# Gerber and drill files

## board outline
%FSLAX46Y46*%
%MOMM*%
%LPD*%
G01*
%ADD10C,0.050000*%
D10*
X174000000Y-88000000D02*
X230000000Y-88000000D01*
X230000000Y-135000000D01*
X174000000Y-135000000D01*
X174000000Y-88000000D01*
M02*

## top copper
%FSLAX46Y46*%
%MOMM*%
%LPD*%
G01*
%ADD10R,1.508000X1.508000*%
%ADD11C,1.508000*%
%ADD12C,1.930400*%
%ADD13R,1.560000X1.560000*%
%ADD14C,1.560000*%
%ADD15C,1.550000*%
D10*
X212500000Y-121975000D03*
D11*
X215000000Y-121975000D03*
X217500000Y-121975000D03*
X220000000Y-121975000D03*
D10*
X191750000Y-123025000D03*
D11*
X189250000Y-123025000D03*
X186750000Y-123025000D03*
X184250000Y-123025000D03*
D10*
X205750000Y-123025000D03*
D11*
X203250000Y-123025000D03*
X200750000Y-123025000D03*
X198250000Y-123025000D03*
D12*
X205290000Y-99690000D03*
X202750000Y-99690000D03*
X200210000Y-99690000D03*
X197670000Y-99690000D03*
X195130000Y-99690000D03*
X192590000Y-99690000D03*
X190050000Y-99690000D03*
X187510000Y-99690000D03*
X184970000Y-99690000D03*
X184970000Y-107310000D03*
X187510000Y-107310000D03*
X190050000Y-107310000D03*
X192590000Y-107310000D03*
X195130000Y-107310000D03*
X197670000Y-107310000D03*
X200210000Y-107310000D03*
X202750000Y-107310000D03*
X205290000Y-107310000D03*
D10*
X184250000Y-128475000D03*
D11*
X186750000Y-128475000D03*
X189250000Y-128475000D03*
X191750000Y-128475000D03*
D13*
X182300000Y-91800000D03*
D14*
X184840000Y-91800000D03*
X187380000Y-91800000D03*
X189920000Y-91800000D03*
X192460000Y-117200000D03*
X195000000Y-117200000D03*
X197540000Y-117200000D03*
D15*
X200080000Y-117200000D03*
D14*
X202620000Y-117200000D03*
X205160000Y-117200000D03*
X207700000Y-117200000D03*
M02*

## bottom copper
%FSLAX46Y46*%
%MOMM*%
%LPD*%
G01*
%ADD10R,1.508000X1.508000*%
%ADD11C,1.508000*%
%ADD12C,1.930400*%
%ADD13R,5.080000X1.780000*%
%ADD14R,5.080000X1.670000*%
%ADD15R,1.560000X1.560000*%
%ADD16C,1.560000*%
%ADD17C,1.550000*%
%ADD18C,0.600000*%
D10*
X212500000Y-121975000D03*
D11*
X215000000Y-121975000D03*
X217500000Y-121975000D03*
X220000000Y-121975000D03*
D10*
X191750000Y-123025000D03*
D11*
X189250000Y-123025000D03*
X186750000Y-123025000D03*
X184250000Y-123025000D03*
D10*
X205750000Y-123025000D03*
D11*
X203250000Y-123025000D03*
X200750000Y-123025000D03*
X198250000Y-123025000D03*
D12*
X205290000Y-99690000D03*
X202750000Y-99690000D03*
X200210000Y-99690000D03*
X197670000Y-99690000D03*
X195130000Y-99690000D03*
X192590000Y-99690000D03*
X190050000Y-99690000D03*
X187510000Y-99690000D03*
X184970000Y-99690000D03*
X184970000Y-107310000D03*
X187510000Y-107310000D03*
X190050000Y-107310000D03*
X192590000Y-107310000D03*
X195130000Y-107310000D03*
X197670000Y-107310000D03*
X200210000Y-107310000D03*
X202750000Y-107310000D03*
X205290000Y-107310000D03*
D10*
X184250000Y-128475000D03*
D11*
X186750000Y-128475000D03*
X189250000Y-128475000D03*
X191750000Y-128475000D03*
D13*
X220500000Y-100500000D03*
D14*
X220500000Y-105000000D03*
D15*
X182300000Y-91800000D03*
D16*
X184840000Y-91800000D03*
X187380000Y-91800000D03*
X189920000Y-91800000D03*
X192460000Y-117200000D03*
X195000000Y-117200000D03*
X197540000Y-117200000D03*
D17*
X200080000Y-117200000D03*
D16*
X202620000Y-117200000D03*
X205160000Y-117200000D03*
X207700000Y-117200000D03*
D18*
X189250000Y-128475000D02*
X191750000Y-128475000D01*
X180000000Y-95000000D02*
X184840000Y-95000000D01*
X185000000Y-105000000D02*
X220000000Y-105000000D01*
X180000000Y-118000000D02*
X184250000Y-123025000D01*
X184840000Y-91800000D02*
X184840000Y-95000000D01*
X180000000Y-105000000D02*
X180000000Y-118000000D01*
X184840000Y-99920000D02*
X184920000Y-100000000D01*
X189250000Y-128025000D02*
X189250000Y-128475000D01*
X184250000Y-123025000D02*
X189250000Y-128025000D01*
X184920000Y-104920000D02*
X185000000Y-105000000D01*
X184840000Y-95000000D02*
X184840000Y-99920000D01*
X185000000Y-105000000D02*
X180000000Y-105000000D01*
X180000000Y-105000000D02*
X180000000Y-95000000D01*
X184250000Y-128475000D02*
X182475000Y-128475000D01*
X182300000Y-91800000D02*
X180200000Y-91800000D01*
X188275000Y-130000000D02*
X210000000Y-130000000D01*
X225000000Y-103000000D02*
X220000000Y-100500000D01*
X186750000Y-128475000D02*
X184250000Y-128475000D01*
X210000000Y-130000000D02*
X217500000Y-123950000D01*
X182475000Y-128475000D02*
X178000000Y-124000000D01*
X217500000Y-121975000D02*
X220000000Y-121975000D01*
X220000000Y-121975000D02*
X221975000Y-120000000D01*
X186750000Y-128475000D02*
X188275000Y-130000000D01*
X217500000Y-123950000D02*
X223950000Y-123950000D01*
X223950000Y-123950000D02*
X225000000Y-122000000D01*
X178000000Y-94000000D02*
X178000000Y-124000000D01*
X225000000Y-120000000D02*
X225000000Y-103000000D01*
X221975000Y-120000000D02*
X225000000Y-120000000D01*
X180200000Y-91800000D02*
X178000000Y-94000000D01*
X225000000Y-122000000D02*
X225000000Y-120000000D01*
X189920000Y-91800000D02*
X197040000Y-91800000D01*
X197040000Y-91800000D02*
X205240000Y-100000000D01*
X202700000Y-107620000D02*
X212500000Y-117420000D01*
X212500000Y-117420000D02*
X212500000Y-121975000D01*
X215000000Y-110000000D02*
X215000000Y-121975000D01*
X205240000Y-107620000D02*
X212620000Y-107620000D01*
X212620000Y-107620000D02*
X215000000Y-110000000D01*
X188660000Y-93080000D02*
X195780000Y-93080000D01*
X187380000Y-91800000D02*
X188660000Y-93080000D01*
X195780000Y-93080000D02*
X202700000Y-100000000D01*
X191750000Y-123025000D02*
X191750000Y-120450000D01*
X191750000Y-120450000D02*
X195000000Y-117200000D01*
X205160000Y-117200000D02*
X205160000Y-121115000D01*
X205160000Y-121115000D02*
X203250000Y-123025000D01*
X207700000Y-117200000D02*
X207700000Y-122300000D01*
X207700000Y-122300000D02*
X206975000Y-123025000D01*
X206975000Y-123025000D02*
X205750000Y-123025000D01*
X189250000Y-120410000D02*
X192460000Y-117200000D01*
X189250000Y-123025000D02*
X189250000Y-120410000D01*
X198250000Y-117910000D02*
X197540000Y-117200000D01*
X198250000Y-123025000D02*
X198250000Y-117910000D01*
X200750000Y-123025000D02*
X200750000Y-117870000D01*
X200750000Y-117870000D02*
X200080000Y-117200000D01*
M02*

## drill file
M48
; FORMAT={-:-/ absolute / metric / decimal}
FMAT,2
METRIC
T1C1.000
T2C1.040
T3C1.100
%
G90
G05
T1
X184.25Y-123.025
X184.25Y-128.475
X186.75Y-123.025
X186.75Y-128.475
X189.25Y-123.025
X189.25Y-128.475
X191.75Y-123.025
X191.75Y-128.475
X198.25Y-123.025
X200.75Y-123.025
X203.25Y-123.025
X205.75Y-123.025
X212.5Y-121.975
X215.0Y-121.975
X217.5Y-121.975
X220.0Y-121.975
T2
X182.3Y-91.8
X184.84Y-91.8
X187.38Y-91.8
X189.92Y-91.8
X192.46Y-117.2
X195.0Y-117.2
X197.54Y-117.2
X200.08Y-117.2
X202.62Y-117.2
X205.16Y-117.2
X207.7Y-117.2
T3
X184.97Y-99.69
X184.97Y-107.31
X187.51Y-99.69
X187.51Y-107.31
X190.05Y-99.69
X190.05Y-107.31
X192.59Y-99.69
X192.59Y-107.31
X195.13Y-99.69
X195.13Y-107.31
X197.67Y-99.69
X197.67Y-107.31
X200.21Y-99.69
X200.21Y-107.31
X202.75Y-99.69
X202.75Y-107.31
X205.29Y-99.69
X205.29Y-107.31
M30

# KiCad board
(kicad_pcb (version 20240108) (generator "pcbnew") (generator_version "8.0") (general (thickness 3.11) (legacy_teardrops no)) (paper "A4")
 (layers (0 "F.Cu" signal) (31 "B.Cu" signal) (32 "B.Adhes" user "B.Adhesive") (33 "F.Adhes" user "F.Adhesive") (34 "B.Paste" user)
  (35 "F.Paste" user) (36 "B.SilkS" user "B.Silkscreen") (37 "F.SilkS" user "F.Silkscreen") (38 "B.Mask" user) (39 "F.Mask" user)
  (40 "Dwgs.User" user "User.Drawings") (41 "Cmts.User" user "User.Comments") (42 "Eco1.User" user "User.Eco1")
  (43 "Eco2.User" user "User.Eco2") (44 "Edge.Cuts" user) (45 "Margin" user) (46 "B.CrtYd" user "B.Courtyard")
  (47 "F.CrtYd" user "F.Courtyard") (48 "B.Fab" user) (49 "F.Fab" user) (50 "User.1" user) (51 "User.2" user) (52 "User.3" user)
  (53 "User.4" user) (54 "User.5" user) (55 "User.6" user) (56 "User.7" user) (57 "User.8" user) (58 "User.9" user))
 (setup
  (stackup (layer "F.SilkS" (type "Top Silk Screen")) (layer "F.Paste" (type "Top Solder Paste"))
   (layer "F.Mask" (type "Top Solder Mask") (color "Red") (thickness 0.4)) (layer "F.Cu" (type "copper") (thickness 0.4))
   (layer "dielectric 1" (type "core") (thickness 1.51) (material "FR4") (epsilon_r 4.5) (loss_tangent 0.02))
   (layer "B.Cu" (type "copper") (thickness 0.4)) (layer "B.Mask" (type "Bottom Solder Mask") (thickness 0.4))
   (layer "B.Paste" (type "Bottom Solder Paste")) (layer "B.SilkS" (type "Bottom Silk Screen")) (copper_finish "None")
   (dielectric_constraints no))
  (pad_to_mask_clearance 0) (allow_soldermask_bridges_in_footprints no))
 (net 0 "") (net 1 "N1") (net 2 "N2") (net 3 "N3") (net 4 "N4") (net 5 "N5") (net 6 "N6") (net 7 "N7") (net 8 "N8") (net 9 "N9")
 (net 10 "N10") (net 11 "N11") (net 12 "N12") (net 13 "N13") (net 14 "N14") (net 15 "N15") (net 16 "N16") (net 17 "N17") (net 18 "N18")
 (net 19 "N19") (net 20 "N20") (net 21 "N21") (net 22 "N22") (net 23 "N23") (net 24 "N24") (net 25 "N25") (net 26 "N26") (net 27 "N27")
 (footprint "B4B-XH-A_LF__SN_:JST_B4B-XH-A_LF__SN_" (layer "F.Cu") (at 216.25 122.5 180)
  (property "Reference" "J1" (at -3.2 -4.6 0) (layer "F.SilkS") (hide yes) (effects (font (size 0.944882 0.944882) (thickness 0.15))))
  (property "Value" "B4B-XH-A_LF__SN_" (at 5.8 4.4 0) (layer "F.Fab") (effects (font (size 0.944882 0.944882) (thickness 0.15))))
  (pad "1" thru_hole rect (at 3.75 0.525 180) (size 1.508 1.508) (drill 1) (layers "*.Cu" "*.Mask") (remove_unused_layers no) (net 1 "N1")
   (solder_mask_margin 0.102))
  (pad "2" thru_hole circle (at 1.25 0.525 180) (size 1.508 1.508) (drill 1) (layers "*.Cu" "*.Mask") (remove_unused_layers no) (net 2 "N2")
   (solder_mask_margin 0.102))
  (pad "3" thru_hole circle (at -1.25 0.525 180) (size 1.508 1.508) (drill 1) (layers "*.Cu" "*.Mask") (remove_unused_layers no)
   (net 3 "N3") (solder_mask_margin 0.102))
  (pad "4" thru_hole circle (at -3.75 0.525 180) (size 1.508 1.508) (drill 1) (layers "*.Cu" "*.Mask") (remove_unused_layers no)
   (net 3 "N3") (solder_mask_margin 0.102)))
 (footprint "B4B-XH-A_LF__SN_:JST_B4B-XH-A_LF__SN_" (layer "F.Cu") (at 188 122.5)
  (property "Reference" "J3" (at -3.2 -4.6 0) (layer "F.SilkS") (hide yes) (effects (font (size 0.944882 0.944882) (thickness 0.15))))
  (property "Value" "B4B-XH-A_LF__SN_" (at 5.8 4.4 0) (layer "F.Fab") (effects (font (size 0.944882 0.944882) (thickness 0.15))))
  (pad "1" thru_hole rect (at 3.75 0.525) (size 1.508 1.508) (drill 1) (layers "*.Cu" "*.Mask") (remove_unused_layers no) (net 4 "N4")
   (solder_mask_margin 0.102))
  (pad "2" thru_hole circle (at 1.25 0.525) (size 1.508 1.508) (drill 1) (layers "*.Cu" "*.Mask") (remove_unused_layers no) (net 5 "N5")
   (solder_mask_margin 0.102))
  (pad "3" thru_hole circle (at -1.25 0.525) (size 1.508 1.508) (drill 1) (layers "*.Cu" "*.Mask") (remove_unused_layers no) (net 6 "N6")
   (solder_mask_margin 0.102))
  (pad "4" thru_hole circle (at -3.75 0.525) (size 1.508 1.508) (drill 1) (layers "*.Cu" "*.Mask") (remove_unused_layers no) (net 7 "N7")
   (solder_mask_margin 0.102)))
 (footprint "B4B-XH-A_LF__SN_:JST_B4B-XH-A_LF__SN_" (layer "F.Cu") (at 202 122.5)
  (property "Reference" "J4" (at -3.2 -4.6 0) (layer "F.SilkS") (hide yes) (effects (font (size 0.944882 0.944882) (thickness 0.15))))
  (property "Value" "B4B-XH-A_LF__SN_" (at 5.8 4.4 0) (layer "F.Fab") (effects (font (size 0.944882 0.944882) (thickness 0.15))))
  (pad "1" thru_hole rect (at 3.75 0.525) (size 1.508 1.508) (drill 1) (layers "*.Cu" "*.Mask") (remove_unused_layers no) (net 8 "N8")
   (solder_mask_margin 0.102))
  (pad "2" thru_hole circle (at 1.25 0.525) (size 1.508 1.508) (drill 1) (layers "*.Cu" "*.Mask") (remove_unused_layers no) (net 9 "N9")
   (solder_mask_margin 0.102))
  (pad "3" thru_hole circle (at -1.25 0.525) (size 1.508 1.508) (drill 1) (layers "*.Cu" "*.Mask") (remove_unused_layers no) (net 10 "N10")
   (solder_mask_margin 0.102))
  (pad "4" thru_hole circle (at -3.75 0.525) (size 1.508 1.508) (drill 1) (layers "*.Cu" "*.Mask") (remove_unused_layers no) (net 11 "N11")
   (solder_mask_margin 0.102)))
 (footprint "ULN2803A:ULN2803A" (layer "F.Cu") (at 196.4 103.5 -90)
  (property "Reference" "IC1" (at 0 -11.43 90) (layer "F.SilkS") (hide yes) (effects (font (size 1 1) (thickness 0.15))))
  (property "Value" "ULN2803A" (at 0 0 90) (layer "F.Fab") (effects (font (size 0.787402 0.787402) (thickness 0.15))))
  (pad "1" thru_hole circle (at -3.81 -8.89 270) (size 1.9304 1.9304) (drill 1.1) (layers "*.Cu" "*.Mask") (remove_unused_layers no)
   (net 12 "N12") (solder_mask_margin 0.102))
  (pad "2" thru_hole circle (at -3.81 -6.35 270) (size 1.9304 1.9304) (drill 1.1) (layers "*.Cu" "*.Mask") (remove_unused_layers no)
   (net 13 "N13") (solder_mask_margin 0.102))
  (pad "3" thru_hole circle (at -3.81 -3.81 270) (size 1.9304 1.9304) (drill 1.1) (layers "*.Cu" "*.Mask") (remove_unused_layers no)
   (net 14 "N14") (solder_mask_margin 0.102))
  (pad "4" thru_hole circle (at -3.81 -1.27 270) (size 1.9304 1.9304) (drill 1.1) (layers "*.Cu" "*.Mask") (remove_unused_layers no)
   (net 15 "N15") (solder_mask_margin 0.102))
  (pad "5" thru_hole circle (at -3.81 1.27 270) (size 1.9304 1.9304) (drill 1.1) (layers "*.Cu" "*.Mask") (remove_unused_layers no)
   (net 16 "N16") (solder_mask_margin 0.102))
  (pad "6" thru_hole circle (at -3.81 3.81 270) (size 1.9304 1.9304) (drill 1.1) (layers "*.Cu" "*.Mask") (remove_unused_layers no)
   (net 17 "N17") (solder_mask_margin 0.102))
  (pad "7" thru_hole circle (at -3.81 6.35 270) (size 1.9304 1.9304) (drill 1.1) (layers "*.Cu" "*.Mask") (remove_unused_layers no)
   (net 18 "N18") (solder_mask_margin 0.102))
  (pad "8" thru_hole circle (at -3.81 8.89 270) (size 1.9304 1.9304) (drill 1.1) (layers "*.Cu" "*.Mask") (remove_unused_layers no)
   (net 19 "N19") (solder_mask_margin 0.102))
  (pad "9" thru_hole circle (at -3.81 11.43 270) (size 1.9304 1.9304) (drill 1.1) (layers "*.Cu" "*.Mask") (remove_unused_layers no)
   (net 7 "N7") (solder_mask_margin 0.102))
  (pad "10" thru_hole circle (at 3.81 11.43 270) (size 1.9304 1.9304) (drill 1.1) (layers "*.Cu" "*.Mask") (remove_unused_layers no)
   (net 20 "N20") (solder_mask_margin 0.102))
  (pad "11" thru_hole circle (at 3.81 8.89 270) (size 1.9304 1.9304) (drill 1.1) (layers "*.Cu" "*.Mask") (remove_unused_layers no)
   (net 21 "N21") (solder_mask_margin 0.102))
  (pad "12" thru_hole circle (at 3.81 6.35 270) (size 1.9304 1.9304) (drill 1.1) (layers "*.Cu" "*.Mask") (remove_unused_layers no)
   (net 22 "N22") (solder_mask_margin 0.102))
  (pad "13" thru_hole circle (at 3.81 3.81 270) (size 1.9304 1.9304) (drill 1.1) (layers "*.Cu" "*.Mask") (remove_unused_layers no)
   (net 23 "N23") (solder_mask_margin 0.102))
  (pad "14" thru_hole circle (at 3.81 1.27 270) (size 1.9304 1.9304) (drill 1.1) (layers "*.Cu" "*.Mask") (remove_unused_layers no)
   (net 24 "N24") (solder_mask_margin 0.102))
  (pad "15" thru_hole circle (at 3.81 -1.27 270) (size 1.9304 1.9304) (drill 1.1) (layers "*.Cu" "*.Mask") (remove_unused_layers no)
   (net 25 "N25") (solder_mask_margin 0.102))
  (pad "16" thru_hole circle (at 3.81 -3.81 270) (size 1.9304 1.9304) (drill 1.1) (layers "*.Cu" "*.Mask") (remove_unused_layers no)
   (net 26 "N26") (solder_mask_margin 0.102))
  (pad "17" thru_hole circle (at 3.81 -6.35 270) (size 1.9304 1.9304) (drill 1.1) (layers "*.Cu" "*.Mask") (remove_unused_layers no)
   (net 1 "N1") (solder_mask_margin 0.102))
  (pad "18" thru_hole circle (at 3.81 -8.89 270) (size 1.9304 1.9304) (drill 1.1) (layers "*.Cu" "*.Mask") (remove_unused_layers no)
   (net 2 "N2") (solder_mask_margin 0.102)))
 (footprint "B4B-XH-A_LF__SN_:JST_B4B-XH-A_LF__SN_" (layer "F.Cu") (at 188 129 180)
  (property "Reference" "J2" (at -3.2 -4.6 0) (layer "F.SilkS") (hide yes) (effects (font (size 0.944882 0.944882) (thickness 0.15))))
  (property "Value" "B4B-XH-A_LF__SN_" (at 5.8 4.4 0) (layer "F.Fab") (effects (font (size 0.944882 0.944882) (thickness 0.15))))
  (pad "1" thru_hole rect (at 3.75 0.525 180) (size 1.508 1.508) (drill 1) (layers "*.Cu" "*.Mask") (remove_unused_layers no) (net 3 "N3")
   (solder_mask_margin 0.102))
  (pad "2" thru_hole circle (at 1.25 0.525 180) (size 1.508 1.508) (drill 1) (layers "*.Cu" "*.Mask") (remove_unused_layers no) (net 3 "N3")
   (solder_mask_margin 0.102))
  (pad "3" thru_hole circle (at -1.25 0.525 180) (size 1.508 1.508) (drill 1) (layers "*.Cu" "*.Mask") (remove_unused_layers no)
   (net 7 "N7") (solder_mask_margin 0.102))
  (pad "4" thru_hole circle (at -3.75 0.525 180) (size 1.508 1.508) (drill 1) (layers "*.Cu" "*.Mask") (remove_unused_layers no)
   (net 7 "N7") (solder_mask_margin 0.102)))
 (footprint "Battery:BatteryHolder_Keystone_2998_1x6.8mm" (layer "B.Cu") (at 220 103 90)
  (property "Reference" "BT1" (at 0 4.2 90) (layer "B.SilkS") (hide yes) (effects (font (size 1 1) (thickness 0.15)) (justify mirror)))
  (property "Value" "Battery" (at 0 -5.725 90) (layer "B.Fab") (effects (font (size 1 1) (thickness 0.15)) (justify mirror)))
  (pad "1" smd rect (at 2.5 0.5 90) (size 1.78 5.08) (layers "B.Cu" "B.Paste" "B.Mask") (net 3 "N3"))
  (pad "2" smd rect (at -2 0.5 90) (size 1.67 5.08) (layers "B.Cu" "B.Paste" "B.Mask") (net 7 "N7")))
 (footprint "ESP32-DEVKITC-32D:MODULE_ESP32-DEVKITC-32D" (layer "B.Cu") (at 202.06 104.5 -90)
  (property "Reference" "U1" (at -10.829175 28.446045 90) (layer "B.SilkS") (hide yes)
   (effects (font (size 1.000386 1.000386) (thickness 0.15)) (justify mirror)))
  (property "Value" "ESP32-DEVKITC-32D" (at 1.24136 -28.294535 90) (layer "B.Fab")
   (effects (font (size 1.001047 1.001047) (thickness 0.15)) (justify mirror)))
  (pad "J2-1" thru_hole rect (at -12.7 19.76 270) (size 1.56 1.56) (drill 1.04) (layers "*.Cu" "*.Mask") (remove_unused_layers no)
   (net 3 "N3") (solder_mask_margin 0.102))
  (pad "J2-2" thru_hole circle (at -12.7 17.22 270) (size 1.56 1.56) (drill 1.04) (layers "*.Cu" "*.Mask") (remove_unused_layers no)
   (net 7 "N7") (solder_mask_margin 0.102))
  (pad "J2-3" thru_hole circle (at -12.7 14.68 270) (size 1.56 1.56) (drill 1.04) (layers "*.Cu" "*.Mask") (remove_unused_layers no)
   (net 13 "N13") (solder_mask_margin 0.102))
  (pad "J2-4" thru_hole circle (at -12.7 12.14 270) (size 1.56 1.56) (drill 1.04) (layers "*.Cu" "*.Mask") (remove_unused_layers no)
   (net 12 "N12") (solder_mask_margin 0.102))
  (pad "J3-5" thru_hole circle (at 12.7 9.6 270) (size 1.56 1.56) (drill 1.04) (layers "*.Cu" "*.Mask") (remove_unused_layers no)
   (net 5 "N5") (solder_mask_margin 0.102))
  (pad "J3-6" thru_hole circle (at 12.7 7.06 270) (size 1.56 1.56) (drill 1.04) (layers "*.Cu" "*.Mask") (remove_unused_layers no)
   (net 4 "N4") (solder_mask_margin 0.102))
  (pad "J3-7" thru_hole circle (at 12.7 4.52 270) (size 1.56 1.56) (drill 1.04) (layers "*.Cu" "*.Mask") (remove_unused_layers no)
   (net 11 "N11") (solder_mask_margin 0.102))
  (pad "J3-8" thru_hole circle (at 12.7 1.98 270) (size 1.55 1.55) (drill 1.04) (layers "*.Cu" "*.Mask") (remove_unused_layers no)
   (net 10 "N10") (solder_mask_margin 0.102))
  (pad "J3-9" thru_hole circle (at 12.7 -0.56 270) (size 1.56 1.56) (drill 1.04) (layers "*.Cu" "*.Mask") (remove_unused_layers no)
   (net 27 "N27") (solder_mask_margin 0.102))
  (pad "J3-10" thru_hole circle (at 12.7 -3.1 270) (size 1.56 1.56) (drill 1.04) (layers "*.Cu" "*.Mask") (remove_unused_layers no)
   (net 9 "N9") (solder_mask_margin 0.102))
  (pad "J3-11" thru_hole circle (at 12.7 -5.64 270) (size 1.56 1.56) (drill 1.04) (layers "*.Cu" "*.Mask") (remove_unused_layers no)
   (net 8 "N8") (solder_mask_margin 0.102)))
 (gr_rect (start 174 88) (end 230 135) (stroke (width 0.05) (type default)) (fill none) (layer "Edge.Cuts"))
 (segment (start 189.25 128.475) (end 191.75 128.475) (width 0.6) (layer "B.Cu") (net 7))
 (segment (start 180 95) (end 184.84 95) (width 0.6) (layer "B.Cu") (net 7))
 (segment (start 185 105) (end 220 105) (width 0.6) (layer "B.Cu") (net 7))
 (segment (start 180 118) (end 184.25 123.025) (width 0.6) (layer "B.Cu") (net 7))
 (segment (start 184.84 91.8) (end 184.84 95) (width 0.6) (layer "B.Cu") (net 7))
 (segment (start 180 105) (end 180 118) (width 0.6) (layer "B.Cu") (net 7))
 (segment (start 184.84 99.92) (end 184.92 100) (width 0.6) (layer "B.Cu") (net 7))
 (segment (start 189.25 128.025) (end 189.25 128.475) (width 0.6) (layer "B.Cu") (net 7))
 (segment (start 184.25 123.025) (end 189.25 128.025) (width 0.6) (layer "B.Cu") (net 7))
 (segment (start 184.92 104.92) (end 185 105) (width 0.6) (layer "B.Cu") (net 7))
 (segment (start 184.84 95) (end 184.84 99.92) (width 0.6) (layer "B.Cu") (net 7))
 (segment (start 185 105) (end 180 105) (width 0.6) (layer "B.Cu") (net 7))
 (segment (start 180 105) (end 180 95) (width 0.6) (layer "B.Cu") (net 7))
 (segment (start 184.25 128.475) (end 182.475 128.475) (width 0.6) (layer "B.Cu") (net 3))
 (segment (start 182.3 91.8) (end 180.2 91.8) (width 0.6) (layer "B.Cu") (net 3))
 (segment (start 188.275 130) (end 210 130) (width 0.6) (layer "B.Cu") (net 3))
 (segment (start 225 103) (end 220 100.5) (width 0.6) (layer "B.Cu") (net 3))
 (segment (start 186.75 128.475) (end 184.25 128.475) (width 0.6) (layer "B.Cu") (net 3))
 (segment (start 210 130) (end 217.5 123.95) (width 0.6) (layer "B.Cu") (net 3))
 (segment (start 182.475 128.475) (end 178 124) (width 0.6) (layer "B.Cu") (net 3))
 (segment (start 217.5 121.975) (end 220 121.975) (width 0.6) (layer "B.Cu") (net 3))
 (segment (start 220 121.975) (end 221.975 120) (width 0.6) (layer "B.Cu") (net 3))
 (segment (start 186.75 128.475) (end 188.275 130) (width 0.6) (layer "B.Cu") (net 3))
 (segment (start 217.5 123.95) (end 223.95 123.95) (width 0.6) (layer "B.Cu") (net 3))
 (segment (start 223.95 123.95) (end 225 122) (width 0.6) (layer "B.Cu") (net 3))
 (segment (start 178 94) (end 178 124) (width 0.6) (layer "B.Cu") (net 3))
 (segment (start 225 120) (end 225 103) (width 0.6) (layer "B.Cu") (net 3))
 (segment (start 221.975 120) (end 225 120) (width 0.6) (layer "B.Cu") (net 3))
 (segment (start 180.2 91.8) (end 178 94) (width 0.6) (layer "B.Cu") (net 3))
 (segment (start 225 122) (end 225 120) (width 0.6) (layer "B.Cu") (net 3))
 (segment (start 189.92 91.8) (end 197.04 91.8) (width 0.6) (layer "B.Cu") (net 12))
 (segment (start 197.04 91.8) (end 205.24 100) (width 0.6) (layer "B.Cu") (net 12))
 (segment (start 202.7 107.62) (end 212.5 117.42) (width 0.6) (layer "B.Cu") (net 1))
 (segment (start 212.5 117.42) (end 212.5 121.975) (width 0.6) (layer "B.Cu") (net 1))
 (segment (start 215 110) (end 215 121.975) (width 0.6) (layer "B.Cu") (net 2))
 (segment (start 205.24 107.62) (end 212.62 107.62) (width 0.6) (layer "B.Cu") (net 2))
 (segment (start 212.62 107.62) (end 215 110) (width 0.6) (layer "B.Cu") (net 2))
 (segment (start 188.66 93.08) (end 195.78 93.08) (width 0.6) (layer "B.Cu") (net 13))
 (segment (start 187.38 91.8) (end 188.66 93.08) (width 0.6) (layer "B.Cu") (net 13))
 (segment (start 195.78 93.08) (end 202.7 100) (width 0.6) (layer "B.Cu") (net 13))
 (segment (start 191.75 123.025) (end 191.75 120.45) (width 0.6) (layer "B.Cu") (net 4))
 (segment (start 191.75 120.45) (end 195 117.2) (width 0.6) (layer "B.Cu") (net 4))
 (segment (start 205.16 117.2) (end 205.16 121.115) (width 0.6) (layer "B.Cu") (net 9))
 (segment (start 205.16 121.115) (end 203.25 123.025) (width 0.6) (layer "B.Cu") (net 9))
 (segment (start 207.7 117.2) (end 207.7 122.3) (width 0.6) (layer "B.Cu") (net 8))
 (segment (start 207.7 122.3) (end 206.975 123.025) (width 0.6) (layer "B.Cu") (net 8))
 (segment (start 206.975 123.025) (end 205.75 123.025) (width 0.6) (layer "B.Cu") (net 8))
 (segment (start 189.25 120.41) (end 192.46 117.2) (width 0.6) (layer "B.Cu") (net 5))
 (segment (start 189.25 123.025) (end 189.25 120.41) (width 0.6) (layer "B.Cu") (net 5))
 (segment (start 198.25 117.91) (end 197.54 117.2) (width 0.6) (layer "B.Cu") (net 11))
 (segment (start 198.25 123.025) (end 198.25 117.91) (width 0.6) (layer "B.Cu") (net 11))
 (segment (start 200.75 123.025) (end 200.75 117.87) (width 0.6) (layer "B.Cu") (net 10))
 (segment (start 200.75 117.87) (end 200.08 117.2) (width 0.6) (layer "B.Cu") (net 10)))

